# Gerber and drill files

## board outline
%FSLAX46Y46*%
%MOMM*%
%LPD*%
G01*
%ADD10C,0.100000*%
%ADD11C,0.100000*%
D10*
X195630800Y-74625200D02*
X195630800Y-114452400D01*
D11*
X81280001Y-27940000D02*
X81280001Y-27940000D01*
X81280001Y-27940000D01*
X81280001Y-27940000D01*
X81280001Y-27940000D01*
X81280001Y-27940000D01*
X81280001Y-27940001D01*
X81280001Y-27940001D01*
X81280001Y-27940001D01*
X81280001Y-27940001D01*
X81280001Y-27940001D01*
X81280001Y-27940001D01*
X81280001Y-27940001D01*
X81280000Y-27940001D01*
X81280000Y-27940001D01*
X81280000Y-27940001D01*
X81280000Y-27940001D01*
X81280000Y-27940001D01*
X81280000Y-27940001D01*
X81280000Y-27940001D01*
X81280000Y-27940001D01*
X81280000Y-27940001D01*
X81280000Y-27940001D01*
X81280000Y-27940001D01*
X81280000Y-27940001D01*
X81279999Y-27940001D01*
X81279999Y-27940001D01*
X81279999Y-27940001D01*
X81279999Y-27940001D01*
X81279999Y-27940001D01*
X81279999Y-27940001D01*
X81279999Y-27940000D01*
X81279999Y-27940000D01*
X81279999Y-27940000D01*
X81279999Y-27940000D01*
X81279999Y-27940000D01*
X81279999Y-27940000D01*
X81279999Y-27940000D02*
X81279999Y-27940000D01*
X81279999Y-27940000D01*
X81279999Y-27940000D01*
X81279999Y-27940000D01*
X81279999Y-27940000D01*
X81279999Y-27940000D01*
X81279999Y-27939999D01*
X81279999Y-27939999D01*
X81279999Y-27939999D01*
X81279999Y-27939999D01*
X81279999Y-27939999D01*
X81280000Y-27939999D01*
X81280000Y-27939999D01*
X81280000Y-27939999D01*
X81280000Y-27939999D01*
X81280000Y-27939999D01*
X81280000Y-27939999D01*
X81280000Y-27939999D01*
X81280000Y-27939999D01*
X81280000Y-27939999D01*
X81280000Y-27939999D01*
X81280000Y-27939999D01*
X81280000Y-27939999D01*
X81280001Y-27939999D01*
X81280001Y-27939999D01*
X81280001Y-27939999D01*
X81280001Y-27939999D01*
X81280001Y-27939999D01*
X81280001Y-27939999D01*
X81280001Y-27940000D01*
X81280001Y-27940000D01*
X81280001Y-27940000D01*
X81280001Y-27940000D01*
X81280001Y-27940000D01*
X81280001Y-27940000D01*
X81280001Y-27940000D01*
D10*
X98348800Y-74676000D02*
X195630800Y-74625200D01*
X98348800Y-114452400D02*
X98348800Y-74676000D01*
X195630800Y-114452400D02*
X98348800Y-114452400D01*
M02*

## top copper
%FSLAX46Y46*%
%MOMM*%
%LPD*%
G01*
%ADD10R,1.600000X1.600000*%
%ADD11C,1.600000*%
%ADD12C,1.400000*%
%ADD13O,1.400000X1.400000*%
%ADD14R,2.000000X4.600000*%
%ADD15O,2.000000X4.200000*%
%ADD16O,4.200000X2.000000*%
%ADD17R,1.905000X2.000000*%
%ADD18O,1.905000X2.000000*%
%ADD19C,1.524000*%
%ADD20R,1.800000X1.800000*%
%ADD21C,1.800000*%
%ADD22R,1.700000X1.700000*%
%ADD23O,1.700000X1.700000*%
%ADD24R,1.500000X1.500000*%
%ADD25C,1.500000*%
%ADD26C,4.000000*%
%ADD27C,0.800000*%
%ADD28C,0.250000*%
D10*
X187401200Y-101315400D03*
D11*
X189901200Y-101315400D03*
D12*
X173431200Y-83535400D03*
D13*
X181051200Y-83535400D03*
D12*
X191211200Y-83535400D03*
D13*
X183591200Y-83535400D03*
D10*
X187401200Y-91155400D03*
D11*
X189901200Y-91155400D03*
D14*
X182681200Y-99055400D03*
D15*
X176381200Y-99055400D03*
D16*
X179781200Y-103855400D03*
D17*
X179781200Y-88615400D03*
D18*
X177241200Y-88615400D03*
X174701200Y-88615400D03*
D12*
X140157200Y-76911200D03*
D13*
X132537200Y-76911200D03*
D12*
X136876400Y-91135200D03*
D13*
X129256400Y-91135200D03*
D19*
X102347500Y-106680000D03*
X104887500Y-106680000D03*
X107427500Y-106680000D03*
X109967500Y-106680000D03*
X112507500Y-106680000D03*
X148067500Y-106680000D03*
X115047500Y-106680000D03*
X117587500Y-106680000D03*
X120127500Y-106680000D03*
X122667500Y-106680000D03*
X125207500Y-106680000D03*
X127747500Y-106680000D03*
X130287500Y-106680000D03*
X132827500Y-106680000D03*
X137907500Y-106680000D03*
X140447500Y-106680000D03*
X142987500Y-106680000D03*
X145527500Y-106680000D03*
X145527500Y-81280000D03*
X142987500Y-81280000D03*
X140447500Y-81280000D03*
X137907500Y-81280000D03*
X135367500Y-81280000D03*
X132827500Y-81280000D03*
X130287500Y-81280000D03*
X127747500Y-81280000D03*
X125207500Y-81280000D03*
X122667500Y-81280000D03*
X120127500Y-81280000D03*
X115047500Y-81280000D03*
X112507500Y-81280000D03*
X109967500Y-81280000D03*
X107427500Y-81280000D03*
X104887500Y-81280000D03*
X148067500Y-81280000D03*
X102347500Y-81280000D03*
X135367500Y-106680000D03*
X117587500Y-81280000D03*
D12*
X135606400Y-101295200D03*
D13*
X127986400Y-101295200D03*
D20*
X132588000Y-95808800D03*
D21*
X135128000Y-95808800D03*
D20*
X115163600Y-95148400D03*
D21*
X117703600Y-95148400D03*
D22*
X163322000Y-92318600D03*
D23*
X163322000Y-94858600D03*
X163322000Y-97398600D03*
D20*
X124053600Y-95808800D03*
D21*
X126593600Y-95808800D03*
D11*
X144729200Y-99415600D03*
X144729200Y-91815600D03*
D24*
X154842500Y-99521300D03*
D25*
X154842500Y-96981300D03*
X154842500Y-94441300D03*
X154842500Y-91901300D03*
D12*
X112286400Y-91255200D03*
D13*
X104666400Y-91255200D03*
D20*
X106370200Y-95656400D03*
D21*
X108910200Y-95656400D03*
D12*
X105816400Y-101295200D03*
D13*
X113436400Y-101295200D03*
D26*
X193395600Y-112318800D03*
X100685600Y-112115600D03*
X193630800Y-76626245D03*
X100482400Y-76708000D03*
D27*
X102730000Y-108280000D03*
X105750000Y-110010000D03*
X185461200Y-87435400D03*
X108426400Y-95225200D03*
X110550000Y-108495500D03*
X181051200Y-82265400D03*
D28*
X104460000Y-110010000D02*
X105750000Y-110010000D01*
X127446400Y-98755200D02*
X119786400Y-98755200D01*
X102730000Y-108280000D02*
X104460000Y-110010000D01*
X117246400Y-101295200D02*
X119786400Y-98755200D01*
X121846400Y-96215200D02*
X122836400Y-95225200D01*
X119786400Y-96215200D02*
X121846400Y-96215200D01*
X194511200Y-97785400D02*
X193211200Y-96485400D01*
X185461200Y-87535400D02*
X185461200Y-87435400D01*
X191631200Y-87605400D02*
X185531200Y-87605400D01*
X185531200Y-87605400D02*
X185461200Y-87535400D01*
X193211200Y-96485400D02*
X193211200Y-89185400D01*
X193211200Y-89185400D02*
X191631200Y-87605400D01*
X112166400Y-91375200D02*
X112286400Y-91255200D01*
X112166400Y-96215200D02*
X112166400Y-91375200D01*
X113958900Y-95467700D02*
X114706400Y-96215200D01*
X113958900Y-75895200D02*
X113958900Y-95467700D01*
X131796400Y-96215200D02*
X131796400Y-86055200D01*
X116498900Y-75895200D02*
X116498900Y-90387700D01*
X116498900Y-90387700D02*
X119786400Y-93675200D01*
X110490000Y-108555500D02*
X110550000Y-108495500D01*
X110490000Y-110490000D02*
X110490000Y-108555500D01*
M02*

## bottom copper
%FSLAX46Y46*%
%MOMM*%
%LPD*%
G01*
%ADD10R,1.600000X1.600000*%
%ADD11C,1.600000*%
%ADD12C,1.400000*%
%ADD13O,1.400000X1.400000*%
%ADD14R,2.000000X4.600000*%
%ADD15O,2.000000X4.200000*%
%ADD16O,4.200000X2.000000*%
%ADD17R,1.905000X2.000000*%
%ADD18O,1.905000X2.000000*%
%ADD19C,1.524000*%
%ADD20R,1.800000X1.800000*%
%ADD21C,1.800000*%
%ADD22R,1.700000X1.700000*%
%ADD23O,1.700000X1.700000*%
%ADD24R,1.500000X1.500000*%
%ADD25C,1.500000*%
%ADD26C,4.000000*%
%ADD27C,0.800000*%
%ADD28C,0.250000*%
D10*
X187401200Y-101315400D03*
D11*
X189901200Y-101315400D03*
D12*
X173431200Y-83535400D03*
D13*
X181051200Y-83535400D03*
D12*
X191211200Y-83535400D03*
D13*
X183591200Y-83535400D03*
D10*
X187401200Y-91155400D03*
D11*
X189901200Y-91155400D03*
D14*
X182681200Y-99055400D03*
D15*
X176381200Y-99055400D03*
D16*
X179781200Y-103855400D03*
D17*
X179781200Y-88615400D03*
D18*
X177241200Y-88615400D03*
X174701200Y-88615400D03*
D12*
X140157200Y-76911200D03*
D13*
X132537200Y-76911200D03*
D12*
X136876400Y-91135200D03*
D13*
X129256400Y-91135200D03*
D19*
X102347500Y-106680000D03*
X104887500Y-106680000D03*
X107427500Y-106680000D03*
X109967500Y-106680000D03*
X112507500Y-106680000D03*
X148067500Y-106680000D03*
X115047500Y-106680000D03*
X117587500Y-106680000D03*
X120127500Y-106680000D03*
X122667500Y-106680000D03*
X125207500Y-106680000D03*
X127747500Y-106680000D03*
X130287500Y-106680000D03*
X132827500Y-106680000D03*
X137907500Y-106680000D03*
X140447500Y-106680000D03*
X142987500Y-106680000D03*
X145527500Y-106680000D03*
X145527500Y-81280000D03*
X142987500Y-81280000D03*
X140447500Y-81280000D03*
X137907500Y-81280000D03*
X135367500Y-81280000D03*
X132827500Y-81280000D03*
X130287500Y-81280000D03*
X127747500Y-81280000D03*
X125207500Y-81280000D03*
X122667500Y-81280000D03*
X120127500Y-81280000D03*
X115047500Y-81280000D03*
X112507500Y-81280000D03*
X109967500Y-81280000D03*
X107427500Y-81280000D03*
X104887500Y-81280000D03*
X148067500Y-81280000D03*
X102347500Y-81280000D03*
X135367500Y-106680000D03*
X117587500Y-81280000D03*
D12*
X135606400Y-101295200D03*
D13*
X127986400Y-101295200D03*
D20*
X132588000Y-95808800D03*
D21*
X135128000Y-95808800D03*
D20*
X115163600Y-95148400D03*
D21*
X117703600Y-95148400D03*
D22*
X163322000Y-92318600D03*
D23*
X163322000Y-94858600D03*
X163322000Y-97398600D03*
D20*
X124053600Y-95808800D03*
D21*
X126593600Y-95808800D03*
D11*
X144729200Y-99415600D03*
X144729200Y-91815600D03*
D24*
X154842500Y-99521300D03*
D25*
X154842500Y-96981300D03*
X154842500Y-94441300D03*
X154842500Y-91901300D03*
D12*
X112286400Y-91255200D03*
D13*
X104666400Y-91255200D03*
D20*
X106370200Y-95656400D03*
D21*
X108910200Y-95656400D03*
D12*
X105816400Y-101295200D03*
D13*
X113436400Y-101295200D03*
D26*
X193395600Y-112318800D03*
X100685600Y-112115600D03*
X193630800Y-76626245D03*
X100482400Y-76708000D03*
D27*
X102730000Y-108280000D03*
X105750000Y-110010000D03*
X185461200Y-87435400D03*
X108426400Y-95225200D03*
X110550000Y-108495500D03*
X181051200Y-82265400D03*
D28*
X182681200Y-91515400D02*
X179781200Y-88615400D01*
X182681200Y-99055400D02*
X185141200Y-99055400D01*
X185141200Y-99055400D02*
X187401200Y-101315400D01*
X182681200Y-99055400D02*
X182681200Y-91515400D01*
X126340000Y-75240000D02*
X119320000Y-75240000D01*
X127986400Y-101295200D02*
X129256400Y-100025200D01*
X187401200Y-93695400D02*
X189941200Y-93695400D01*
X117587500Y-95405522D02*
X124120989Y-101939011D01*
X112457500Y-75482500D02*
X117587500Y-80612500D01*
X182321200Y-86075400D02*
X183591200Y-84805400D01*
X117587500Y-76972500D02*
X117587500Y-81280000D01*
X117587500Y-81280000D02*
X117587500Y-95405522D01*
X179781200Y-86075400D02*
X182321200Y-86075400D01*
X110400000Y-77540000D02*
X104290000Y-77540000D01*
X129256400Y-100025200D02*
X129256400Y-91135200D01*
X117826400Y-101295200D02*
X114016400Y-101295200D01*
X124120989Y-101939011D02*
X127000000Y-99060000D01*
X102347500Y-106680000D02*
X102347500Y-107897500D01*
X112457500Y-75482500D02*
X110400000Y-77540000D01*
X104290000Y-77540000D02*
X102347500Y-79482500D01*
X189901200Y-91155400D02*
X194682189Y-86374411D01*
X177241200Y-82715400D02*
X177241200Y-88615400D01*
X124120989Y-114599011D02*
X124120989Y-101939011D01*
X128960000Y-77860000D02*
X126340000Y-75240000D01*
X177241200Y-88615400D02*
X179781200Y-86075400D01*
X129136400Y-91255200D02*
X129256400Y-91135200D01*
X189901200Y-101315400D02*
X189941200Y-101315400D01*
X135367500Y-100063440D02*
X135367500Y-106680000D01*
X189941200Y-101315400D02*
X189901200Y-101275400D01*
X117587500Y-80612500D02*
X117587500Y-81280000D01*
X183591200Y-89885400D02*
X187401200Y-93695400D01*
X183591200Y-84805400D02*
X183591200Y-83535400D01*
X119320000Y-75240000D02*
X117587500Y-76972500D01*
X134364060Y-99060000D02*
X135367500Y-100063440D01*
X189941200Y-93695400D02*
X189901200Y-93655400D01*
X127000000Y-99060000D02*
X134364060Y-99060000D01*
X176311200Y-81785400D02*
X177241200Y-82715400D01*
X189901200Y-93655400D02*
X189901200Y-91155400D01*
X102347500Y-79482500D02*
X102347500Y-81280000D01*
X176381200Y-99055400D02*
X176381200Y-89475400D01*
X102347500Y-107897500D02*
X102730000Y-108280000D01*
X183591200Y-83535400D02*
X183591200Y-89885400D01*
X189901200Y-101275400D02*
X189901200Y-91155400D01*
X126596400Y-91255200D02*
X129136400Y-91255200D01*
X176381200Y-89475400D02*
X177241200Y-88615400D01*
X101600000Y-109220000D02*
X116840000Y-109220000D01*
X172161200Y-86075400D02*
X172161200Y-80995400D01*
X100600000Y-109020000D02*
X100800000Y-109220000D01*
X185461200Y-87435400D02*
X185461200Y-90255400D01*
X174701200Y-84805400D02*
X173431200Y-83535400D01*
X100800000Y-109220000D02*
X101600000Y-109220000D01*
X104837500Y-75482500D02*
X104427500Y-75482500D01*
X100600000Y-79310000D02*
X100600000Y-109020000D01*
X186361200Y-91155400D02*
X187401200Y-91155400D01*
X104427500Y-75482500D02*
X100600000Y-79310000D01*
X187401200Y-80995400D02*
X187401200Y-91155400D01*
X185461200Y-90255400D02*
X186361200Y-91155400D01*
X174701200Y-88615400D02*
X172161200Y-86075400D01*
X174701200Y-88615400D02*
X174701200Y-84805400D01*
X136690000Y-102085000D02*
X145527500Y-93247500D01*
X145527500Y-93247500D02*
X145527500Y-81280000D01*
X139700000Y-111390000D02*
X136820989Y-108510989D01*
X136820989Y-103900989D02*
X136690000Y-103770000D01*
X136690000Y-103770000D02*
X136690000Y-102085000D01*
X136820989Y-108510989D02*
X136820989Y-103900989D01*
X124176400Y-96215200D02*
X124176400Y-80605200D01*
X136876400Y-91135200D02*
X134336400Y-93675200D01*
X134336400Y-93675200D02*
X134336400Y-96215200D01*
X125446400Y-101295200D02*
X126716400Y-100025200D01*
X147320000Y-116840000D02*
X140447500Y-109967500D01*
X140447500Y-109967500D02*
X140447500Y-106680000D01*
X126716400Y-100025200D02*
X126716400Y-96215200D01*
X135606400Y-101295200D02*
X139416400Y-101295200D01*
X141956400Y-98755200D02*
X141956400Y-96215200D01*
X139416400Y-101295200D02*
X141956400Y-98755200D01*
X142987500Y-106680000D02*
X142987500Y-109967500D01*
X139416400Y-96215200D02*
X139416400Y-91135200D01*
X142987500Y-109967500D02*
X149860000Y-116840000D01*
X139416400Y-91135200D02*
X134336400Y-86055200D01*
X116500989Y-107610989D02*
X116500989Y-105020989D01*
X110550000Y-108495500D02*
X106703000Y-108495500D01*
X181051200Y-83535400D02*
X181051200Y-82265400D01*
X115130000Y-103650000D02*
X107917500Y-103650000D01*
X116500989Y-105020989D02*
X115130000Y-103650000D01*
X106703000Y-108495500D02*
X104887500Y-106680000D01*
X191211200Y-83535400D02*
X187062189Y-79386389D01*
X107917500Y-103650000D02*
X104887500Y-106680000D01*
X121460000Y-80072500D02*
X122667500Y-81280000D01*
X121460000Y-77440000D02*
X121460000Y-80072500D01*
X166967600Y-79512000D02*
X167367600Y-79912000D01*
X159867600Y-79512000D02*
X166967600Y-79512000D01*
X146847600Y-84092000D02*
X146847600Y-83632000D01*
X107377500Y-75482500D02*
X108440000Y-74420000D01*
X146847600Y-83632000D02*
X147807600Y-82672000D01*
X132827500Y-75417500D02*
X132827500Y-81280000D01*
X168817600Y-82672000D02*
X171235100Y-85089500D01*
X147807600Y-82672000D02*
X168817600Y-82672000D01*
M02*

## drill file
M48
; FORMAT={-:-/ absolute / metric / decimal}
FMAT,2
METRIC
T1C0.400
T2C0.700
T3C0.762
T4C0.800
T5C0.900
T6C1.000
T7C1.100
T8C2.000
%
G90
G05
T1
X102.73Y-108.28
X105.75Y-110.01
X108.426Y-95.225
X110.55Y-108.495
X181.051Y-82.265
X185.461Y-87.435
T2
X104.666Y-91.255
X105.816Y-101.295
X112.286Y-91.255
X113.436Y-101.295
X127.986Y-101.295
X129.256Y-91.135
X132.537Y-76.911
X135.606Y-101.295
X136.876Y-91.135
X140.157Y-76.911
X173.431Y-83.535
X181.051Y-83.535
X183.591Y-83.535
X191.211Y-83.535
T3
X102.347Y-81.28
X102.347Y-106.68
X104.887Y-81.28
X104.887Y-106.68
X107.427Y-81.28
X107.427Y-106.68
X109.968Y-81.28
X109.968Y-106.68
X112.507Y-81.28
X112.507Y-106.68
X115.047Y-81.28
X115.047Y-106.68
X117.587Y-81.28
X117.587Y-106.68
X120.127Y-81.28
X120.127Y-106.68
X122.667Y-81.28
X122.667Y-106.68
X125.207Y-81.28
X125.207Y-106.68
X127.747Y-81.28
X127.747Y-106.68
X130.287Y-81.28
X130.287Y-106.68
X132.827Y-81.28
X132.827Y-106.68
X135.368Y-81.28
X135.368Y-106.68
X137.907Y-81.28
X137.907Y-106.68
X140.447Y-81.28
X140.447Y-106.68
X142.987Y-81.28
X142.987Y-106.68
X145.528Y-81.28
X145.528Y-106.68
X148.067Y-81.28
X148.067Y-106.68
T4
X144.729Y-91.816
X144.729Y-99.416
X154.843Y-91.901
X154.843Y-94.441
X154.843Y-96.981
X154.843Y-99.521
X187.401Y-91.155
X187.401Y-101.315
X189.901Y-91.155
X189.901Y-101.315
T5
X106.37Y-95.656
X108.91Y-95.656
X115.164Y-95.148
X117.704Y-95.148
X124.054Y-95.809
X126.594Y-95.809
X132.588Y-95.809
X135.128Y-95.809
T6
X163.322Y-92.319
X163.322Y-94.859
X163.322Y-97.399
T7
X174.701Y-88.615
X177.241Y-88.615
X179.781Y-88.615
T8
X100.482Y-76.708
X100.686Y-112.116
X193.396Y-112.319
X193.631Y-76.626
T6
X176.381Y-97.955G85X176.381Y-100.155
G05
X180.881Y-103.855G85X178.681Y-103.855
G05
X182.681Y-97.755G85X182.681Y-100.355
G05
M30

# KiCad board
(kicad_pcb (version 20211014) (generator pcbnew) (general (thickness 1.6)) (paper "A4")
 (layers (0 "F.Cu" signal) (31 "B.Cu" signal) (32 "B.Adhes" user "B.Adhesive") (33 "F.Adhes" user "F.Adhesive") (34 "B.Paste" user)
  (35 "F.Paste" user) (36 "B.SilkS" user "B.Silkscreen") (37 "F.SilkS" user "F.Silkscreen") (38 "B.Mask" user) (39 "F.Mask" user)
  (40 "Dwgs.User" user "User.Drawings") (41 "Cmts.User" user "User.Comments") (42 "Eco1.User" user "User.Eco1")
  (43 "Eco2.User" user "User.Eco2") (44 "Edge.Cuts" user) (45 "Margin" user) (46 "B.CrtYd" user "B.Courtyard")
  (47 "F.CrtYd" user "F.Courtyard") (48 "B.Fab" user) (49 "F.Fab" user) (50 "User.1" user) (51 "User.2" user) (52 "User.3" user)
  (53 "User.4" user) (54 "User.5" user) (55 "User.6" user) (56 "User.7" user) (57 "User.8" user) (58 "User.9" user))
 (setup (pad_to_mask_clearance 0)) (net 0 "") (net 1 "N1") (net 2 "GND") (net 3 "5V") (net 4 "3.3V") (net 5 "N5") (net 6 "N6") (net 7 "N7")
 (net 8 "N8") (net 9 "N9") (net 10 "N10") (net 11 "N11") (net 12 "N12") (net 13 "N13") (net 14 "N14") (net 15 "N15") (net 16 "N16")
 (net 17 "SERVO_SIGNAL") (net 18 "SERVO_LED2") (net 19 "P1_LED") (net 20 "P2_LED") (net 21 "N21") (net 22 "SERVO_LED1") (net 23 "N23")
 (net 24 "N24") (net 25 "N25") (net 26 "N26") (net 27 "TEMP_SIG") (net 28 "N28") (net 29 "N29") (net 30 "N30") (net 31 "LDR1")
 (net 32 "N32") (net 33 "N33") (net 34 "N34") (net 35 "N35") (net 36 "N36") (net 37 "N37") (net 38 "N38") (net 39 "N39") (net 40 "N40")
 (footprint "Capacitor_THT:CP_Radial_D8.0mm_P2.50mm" (layer "F.Cu") (at 187.4012 101.3154)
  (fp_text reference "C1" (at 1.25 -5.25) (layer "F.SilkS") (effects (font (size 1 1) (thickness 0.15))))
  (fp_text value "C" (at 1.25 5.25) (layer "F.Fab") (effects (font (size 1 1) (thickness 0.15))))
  (pad "1" thru_hole rect (at 0 0) (size 1.6 1.6) (drill 0.8) (layers *.Cu *.Mask) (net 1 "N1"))
  (pad "2" thru_hole circle (at 2.5 0) (size 1.6 1.6) (drill 0.8) (layers *.Cu *.Mask) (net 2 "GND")))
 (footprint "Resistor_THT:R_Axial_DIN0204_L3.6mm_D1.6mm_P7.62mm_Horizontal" (layer "F.Cu") (at 173.4312 83.5354)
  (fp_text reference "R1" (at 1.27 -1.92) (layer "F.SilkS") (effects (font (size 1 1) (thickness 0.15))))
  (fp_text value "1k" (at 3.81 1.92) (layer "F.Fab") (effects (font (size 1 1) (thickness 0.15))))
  (pad "1" thru_hole circle (at 0 0) (size 1.4 1.4) (drill 0.7) (layers *.Cu *.Mask) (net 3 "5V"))
  (pad "2" thru_hole oval (at 7.62 0) (size 1.4 1.4) (drill 0.7) (layers *.Cu *.Mask) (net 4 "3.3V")))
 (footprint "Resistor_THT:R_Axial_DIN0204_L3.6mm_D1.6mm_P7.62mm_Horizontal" (layer "F.Cu") (at 191.2112 83.5354 180)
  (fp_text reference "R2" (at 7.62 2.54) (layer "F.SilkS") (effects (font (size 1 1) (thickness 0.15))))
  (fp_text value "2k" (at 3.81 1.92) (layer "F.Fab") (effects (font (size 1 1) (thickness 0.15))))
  (pad "1" thru_hole circle (at 0 0 180) (size 1.4 1.4) (drill 0.7) (layers *.Cu *.Mask) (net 4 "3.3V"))
  (pad "2" thru_hole oval (at 7.62 0 180) (size 1.4 1.4) (drill 0.7) (layers *.Cu *.Mask) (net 2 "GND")))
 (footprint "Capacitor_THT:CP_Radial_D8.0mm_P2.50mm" (layer "F.Cu") (at 187.4012 91.1554)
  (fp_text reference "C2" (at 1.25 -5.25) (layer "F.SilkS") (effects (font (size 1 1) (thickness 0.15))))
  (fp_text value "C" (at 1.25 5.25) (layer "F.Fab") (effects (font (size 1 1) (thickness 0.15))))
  (pad "1" thru_hole rect (at 0 0) (size 1.6 1.6) (drill 0.8) (layers *.Cu *.Mask) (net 3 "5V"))
  (pad "2" thru_hole circle (at 2.5 0) (size 1.6 1.6) (drill 0.8) (layers *.Cu *.Mask) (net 2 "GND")))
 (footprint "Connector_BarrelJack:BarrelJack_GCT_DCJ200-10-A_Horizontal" (layer "F.Cu") (at 182.6812 99.0554 -90)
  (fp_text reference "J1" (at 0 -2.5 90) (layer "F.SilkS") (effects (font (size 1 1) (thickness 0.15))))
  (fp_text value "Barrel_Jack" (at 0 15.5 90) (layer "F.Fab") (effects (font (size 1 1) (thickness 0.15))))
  (pad "1" thru_hole rect (at 0 0 270) (size 4.6 2) (drill oval 3.6 1) (layers *.Cu *.Mask) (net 1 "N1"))
  (pad "2" thru_hole oval (at 0 6.3 270) (size 4.2 2) (drill oval 3.2 1) (layers *.Cu *.Mask) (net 2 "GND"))
  (pad "3" thru_hole oval (at 4.8 2.9 270) (size 2 4.2) (drill oval 1 3.2) (layers *.Cu *.Mask)))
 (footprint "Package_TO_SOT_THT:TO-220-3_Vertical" (layer "F.Cu") (at 179.7812 88.6154 180)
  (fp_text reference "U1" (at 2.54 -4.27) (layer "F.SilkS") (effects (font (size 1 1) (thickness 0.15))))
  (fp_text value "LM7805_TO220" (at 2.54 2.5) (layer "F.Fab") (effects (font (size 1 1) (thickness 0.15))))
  (pad "1" thru_hole rect (at 0 0 180) (size 1.905 2) (drill 1.1) (layers *.Cu *.Mask) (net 1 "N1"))
  (pad "2" thru_hole oval (at 2.54 0 180) (size 1.905 2) (drill 1.1) (layers *.Cu *.Mask) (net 2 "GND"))
  (pad "3" thru_hole oval (at 5.08 0 180) (size 1.905 2) (drill 1.1) (layers *.Cu *.Mask) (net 3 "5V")))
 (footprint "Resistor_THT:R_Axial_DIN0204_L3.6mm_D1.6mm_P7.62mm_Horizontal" (layer "F.Cu") (at 140.1572 76.9112 180)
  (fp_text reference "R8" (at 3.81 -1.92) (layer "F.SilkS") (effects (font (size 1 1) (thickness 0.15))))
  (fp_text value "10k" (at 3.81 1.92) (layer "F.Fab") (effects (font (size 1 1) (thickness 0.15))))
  (pad "1" thru_hole circle (at 0 0 180) (size 1.4 1.4) (drill 0.7) (layers *.Cu *.Mask) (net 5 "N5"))
  (pad "2" thru_hole oval (at 7.62 0 180) (size 1.4 1.4) (drill 0.7) (layers *.Cu *.Mask) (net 2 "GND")))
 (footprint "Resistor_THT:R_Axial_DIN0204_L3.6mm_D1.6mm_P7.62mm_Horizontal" (layer "F.Cu") (at 136.8764 91.1352 180)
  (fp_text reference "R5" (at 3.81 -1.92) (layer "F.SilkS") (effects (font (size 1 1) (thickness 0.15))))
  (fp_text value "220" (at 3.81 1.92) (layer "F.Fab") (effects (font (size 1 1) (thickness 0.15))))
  (pad "1" thru_hole circle (at 0 0 180) (size 1.4 1.4) (drill 0.7) (layers *.Cu *.Mask) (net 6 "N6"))
  (pad "2" thru_hole oval (at 7.62 0 180) (size 1.4 1.4) (drill 0.7) (layers *.Cu *.Mask) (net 2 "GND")))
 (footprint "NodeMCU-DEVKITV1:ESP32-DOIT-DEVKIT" (layer "F.Cu") (at 99.8075 93.98 90)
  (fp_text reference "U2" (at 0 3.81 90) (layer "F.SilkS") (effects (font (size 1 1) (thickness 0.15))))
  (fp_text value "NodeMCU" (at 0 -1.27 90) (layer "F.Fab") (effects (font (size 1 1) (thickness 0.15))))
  (pad "1" thru_hole circle (at -12.7 2.54 90) (size 1.524 1.524) (drill 0.762) (layers *.Cu *.Mask) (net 2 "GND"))
  (pad "2" thru_hole circle (at -12.7 5.08 90) (size 1.524 1.524) (drill 0.762) (layers *.Cu *.Mask) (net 4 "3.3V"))
  (pad "3" thru_hole circle (at -12.7 7.62 90) (size 1.524 1.524) (drill 0.762) (layers *.Cu *.Mask) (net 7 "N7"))
  (pad "4" thru_hole circle (at -12.7 10.16 90) (size 1.524 1.524) (drill 0.762) (layers *.Cu *.Mask) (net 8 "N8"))
  (pad "5" thru_hole circle (at -12.7 12.7 90) (size 1.524 1.524) (drill 0.762) (layers *.Cu *.Mask) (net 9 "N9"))
  (pad "5V" thru_hole circle (at -12.7 48.26 90) (size 1.524 1.524) (drill 0.762) (layers *.Cu *.Mask) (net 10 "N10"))
  (pad "6" thru_hole circle (at -12.7 15.24 90) (size 1.524 1.524) (drill 0.762) (layers *.Cu *.Mask) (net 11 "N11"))
  (pad "7" thru_hole circle (at -12.7 17.78 90) (size 1.524 1.524) (drill 0.762) (layers *.Cu *.Mask) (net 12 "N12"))
  (pad "8" thru_hole circle (at -12.7 20.32 90) (size 1.524 1.524) (drill 0.762) (layers *.Cu *.Mask) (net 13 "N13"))
  (pad "9" thru_hole circle (at -12.7 22.86 90) (size 1.524 1.524) (drill 0.762) (layers *.Cu *.Mask) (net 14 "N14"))
  (pad "10" thru_hole circle (at -12.7 25.4 90) (size 1.524 1.524) (drill 0.762) (layers *.Cu *.Mask) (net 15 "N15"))
  (pad "11" thru_hole circle (at -12.7 27.94 90) (size 1.524 1.524) (drill 0.762) (layers *.Cu *.Mask) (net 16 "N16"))
  (pad "12" thru_hole circle (at -12.7 30.48 90) (size 1.524 1.524) (drill 0.762) (layers *.Cu *.Mask) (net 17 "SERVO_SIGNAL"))
  (pad "13" thru_hole circle (at -12.7 33.02 90) (size 1.524 1.524) (drill 0.762) (layers *.Cu *.Mask) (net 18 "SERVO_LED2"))
  (pad "15" thru_hole circle (at -12.7 38.1 90) (size 1.524 1.524) (drill 0.762) (layers *.Cu *.Mask))
  (pad "16" thru_hole circle (at -12.7 40.64 90) (size 1.524 1.524) (drill 0.762) (layers *.Cu *.Mask) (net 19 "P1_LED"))
  (pad "17" thru_hole circle (at -12.7 43.18 90) (size 1.524 1.524) (drill 0.762) (layers *.Cu *.Mask) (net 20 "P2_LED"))
  (pad "18" thru_hole circle (at -12.7 45.72 90) (size 1.524 1.524) (drill 0.762) (layers *.Cu *.Mask) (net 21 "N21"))
  (pad "19" thru_hole circle (at 12.7 45.72 90) (size 1.524 1.524) (drill 0.762) (layers *.Cu *.Mask) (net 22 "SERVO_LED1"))
  (pad "20" thru_hole circle (at 12.7 43.18 90) (size 1.524 1.524) (drill 0.762) (layers *.Cu *.Mask) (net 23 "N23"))
  (pad "21" thru_hole circle (at 12.7 40.64 90) (size 1.524 1.524) (drill 0.762) (layers *.Cu *.Mask) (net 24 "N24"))
  (pad "22" thru_hole circle (at 12.7 38.1 90) (size 1.524 1.524) (drill 0.762) (layers *.Cu *.Mask) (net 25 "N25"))
  (pad "23" thru_hole circle (at 12.7 35.56 90) (size 1.524 1.524) (drill 0.762) (layers *.Cu *.Mask) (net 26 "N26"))
  (pad "24" thru_hole circle (at 12.7 33.02 90) (size 1.524 1.524) (drill 0.762) (layers *.Cu *.Mask) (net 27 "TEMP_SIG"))
  (pad "25" thru_hole circle (at 12.7 30.48 90) (size 1.524 1.524) (drill 0.762) (layers *.Cu *.Mask) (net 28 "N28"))
  (pad "26" thru_hole circle (at 12.7 27.94 90) (size 1.524 1.524) (drill 0.762) (layers *.Cu *.Mask) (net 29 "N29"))
  (pad "27" thru_hole circle (at 12.7 25.4 90) (size 1.524 1.524) (drill 0.762) (layers *.Cu *.Mask) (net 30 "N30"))
  (pad "28" thru_hole circle (at 12.7 22.86 90) (size 1.524 1.524) (drill 0.762) (layers *.Cu *.Mask) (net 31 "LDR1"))
  (pad "29" thru_hole circle (at 12.7 20.32 90) (size 1.524 1.524) (drill 0.762) (layers *.Cu *.Mask) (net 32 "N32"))
  (pad "31" thru_hole circle (at 12.7 15.24 90) (size 1.524 1.524) (drill 0.762) (layers *.Cu *.Mask) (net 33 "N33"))
  (pad "32" thru_hole circle (at 12.7 12.7 90) (size 1.524 1.524) (drill 0.762) (layers *.Cu *.Mask))
  (pad "33" thru_hole circle (at 12.7 10.16 90) (size 1.524 1.524) (drill 0.762) (layers *.Cu *.Mask) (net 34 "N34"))
  (pad "34" thru_hole circle (at 12.7 7.62 90) (size 1.524 1.524) (drill 0.762) (layers *.Cu *.Mask) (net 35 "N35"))
  (pad "35" thru_hole circle (at 12.7 5.08 90) (size 1.524 1.524) (drill 0.762) (layers *.Cu *.Mask) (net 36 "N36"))
  (pad "38" thru_hole circle (at 12.7 48.26 90) (size 1.524 1.524) (drill 0.762) (layers *.Cu *.Mask))
  (pad "GND" thru_hole circle (at 12.7 2.54 90) (size 1.524 1.524) (drill 0.762) (layers *.Cu *.Mask) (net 2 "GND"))
  (pad "GND" thru_hole circle (at -12.7 35.56 90) (size 1.524 1.524) (drill 0.762) (layers *.Cu *.Mask) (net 2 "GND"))
  (pad "GND" thru_hole circle (at 12.7 17.78 90) (size 1.524 1.524) (drill 0.762) (layers *.Cu *.Mask) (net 2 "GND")))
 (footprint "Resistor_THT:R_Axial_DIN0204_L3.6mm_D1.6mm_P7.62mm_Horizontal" (layer "F.Cu") (at 135.6064 101.2952 180)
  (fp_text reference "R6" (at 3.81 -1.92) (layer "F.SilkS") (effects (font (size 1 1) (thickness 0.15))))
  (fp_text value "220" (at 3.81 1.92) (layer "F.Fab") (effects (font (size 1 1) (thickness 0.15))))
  (pad "1" thru_hole circle (at 0 0 180) (size 1.4 1.4) (drill 0.7) (layers *.Cu *.Mask) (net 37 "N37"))
  (pad "2" thru_hole oval (at 7.62 0 180) (size 1.4 1.4) (drill 0.7) (layers *.Cu *.Mask) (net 2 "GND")))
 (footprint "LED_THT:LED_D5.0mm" (layer "B.Cu") (at 132.588 95.8088)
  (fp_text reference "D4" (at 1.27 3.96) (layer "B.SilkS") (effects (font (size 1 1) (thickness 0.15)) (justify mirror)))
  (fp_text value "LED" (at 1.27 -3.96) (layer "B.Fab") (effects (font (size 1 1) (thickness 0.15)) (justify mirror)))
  (pad "1" thru_hole rect (at 0 0) (size 1.8 1.8) (drill 0.9) (layers *.Cu *.Mask) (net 37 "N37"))
  (pad "2" thru_hole circle (at 2.54 0) (size 1.8 1.8) (drill 0.9) (layers *.Cu *.Mask) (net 20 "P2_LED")))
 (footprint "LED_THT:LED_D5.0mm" (layer "B.Cu") (at 115.1636 95.1484)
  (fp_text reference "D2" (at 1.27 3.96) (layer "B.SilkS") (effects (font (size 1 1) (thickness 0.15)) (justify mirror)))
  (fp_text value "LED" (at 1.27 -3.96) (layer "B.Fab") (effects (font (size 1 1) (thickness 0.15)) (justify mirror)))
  (pad "1" thru_hole rect (at 0 0) (size 1.8 1.8) (drill 0.9) (layers *.Cu *.Mask) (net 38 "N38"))
  (pad "2" thru_hole circle (at 2.54 0) (size 1.8 1.8) (drill 0.9) (layers *.Cu *.Mask) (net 22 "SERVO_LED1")))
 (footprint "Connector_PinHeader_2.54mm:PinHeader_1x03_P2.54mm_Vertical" (layer "B.Cu") (at 163.322 92.3186 180)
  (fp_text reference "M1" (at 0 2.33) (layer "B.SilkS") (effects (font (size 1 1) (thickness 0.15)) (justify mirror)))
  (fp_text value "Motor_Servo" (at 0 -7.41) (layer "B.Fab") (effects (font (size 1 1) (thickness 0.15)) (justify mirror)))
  (pad "1" thru_hole rect (at 0 0 180) (size 1.7 1.7) (drill 1) (layers *.Cu *.Mask) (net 17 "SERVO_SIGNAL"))
  (pad "2" thru_hole oval (at 0 -2.54 180) (size 1.7 1.7) (drill 1) (layers *.Cu *.Mask) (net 3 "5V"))
  (pad "3" thru_hole oval (at 0 -5.08 180) (size 1.7 1.7) (drill 1) (layers *.Cu *.Mask) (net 2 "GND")))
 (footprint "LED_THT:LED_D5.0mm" (layer "B.Cu") (at 124.0536 95.8088)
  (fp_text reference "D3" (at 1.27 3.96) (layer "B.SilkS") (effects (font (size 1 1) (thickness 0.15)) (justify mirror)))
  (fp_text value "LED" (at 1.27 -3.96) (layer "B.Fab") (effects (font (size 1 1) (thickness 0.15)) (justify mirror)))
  (pad "1" thru_hole rect (at 0 0) (size 1.8 1.8) (drill 0.9) (layers *.Cu *.Mask) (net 6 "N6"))
  (pad "2" thru_hole circle (at 2.54 0) (size 1.8 1.8) (drill 0.9) (layers *.Cu *.Mask) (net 19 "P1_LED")))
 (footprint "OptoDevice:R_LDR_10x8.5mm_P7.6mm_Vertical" (layer "B.Cu") (at 144.7292 99.4156 90)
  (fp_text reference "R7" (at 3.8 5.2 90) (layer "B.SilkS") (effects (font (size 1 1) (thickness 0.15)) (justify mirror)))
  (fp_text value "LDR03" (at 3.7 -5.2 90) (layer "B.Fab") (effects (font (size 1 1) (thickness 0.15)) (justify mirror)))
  (pad "1" thru_hole circle (at 0 0 90) (size 1.6 1.6) (drill 0.8) (layers *.Cu *.Mask) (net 31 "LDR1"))
  (pad "2" thru_hole circle (at 7.6 0 90) (size 1.6 1.6) (drill 0.8) (layers *.Cu *.Mask) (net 5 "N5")))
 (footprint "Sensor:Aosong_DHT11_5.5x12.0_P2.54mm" (layer "B.Cu") (at 154.8425 99.5213)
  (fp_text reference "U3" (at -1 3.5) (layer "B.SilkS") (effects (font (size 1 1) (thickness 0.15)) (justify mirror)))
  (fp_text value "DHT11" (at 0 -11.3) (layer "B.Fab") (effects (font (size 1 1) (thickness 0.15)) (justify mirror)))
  (pad "1" thru_hole rect (at 0 0) (size 1.5 1.5) (drill 0.8) (layers *.Cu *.Mask) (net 3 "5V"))
  (pad "2" thru_hole circle (at 0 -2.54) (size 1.5 1.5) (drill 0.8) (layers *.Cu *.Mask) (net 27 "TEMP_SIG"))
  (pad "3" thru_hole circle (at 0 -5.08) (size 1.5 1.5) (drill 0.8) (layers *.Cu *.Mask) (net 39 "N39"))
  (pad "4" thru_hole circle (at 0 -7.62) (size 1.5 1.5) (drill 0.8) (layers *.Cu *.Mask) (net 2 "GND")))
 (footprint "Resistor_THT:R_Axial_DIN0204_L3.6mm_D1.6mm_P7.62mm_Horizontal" (layer "B.Cu") (at 112.2864 91.2552 180)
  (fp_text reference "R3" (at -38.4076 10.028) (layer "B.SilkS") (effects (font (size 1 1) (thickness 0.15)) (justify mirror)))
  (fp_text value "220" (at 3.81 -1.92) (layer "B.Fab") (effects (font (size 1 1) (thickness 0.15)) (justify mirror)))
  (pad "1" thru_hole circle (at 0 0 180) (size 1.4 1.4) (drill 0.7) (layers *.Cu *.Mask) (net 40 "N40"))
  (pad "2" thru_hole oval (at 7.62 0 180) (size 1.4 1.4) (drill 0.7) (layers *.Cu *.Mask) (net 2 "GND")))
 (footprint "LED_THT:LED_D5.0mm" (layer "B.Cu") (at 106.3702 95.6564)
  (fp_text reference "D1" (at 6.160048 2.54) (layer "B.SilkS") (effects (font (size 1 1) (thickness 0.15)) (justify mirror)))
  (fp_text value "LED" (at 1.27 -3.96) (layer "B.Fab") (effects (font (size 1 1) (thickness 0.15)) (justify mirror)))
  (pad "1" thru_hole rect (at 0 0) (size 1.8 1.8) (drill 0.9) (layers *.Cu *.Mask) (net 40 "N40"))
  (pad "2" thru_hole circle (at 2.54 0) (size 1.8 1.8) (drill 0.9) (layers *.Cu *.Mask) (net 18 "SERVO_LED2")))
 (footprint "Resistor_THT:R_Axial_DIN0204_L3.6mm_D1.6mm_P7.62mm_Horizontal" (layer "B.Cu") (at 105.8164 101.2952)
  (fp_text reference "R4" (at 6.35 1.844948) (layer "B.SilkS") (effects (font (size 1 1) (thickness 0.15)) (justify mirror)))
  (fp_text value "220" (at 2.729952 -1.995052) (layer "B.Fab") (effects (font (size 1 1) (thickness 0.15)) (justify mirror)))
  (pad "1" thru_hole circle (at 0 0) (size 1.4 1.4) (drill 0.7) (layers *.Cu *.Mask) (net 38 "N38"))
  (pad "2" thru_hole oval (at 7.62 0) (size 1.4 1.4) (drill 0.7) (layers *.Cu *.Mask) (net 2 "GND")))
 (gr_line (start 195.6308 74.6252) (end 195.6308 114.4524) (layer "Edge.Cuts") (width 0.1))
 (gr_arc (start 81.28 27.94) (mid 81.28 27.94) (end 81.28 27.94) (layer "Edge.Cuts") (width 0.1))
 (gr_line (start 98.3488 74.676) (end 195.6308 74.6252) (layer "Edge.Cuts") (width 0.1))
 (gr_line (start 98.3488 114.4524) (end 98.3488 74.676) (layer "Edge.Cuts") (width 0.1))
 (gr_line (start 195.6308 114.4524) (end 98.3488 114.4524) (layer "Edge.Cuts") (width 0.1))
 (via (at 193.3956 112.3188) (size 4) (drill 2) (layers "F.Cu" "B.Cu") (free) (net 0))
 (via (at 100.6856 112.1156) (size 4) (drill 2) (layers "F.Cu" "B.Cu") (free) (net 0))
 (via (at 193.6308 76.626245) (size 4) (drill 2) (layers "F.Cu" "B.Cu") (free) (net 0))
 (via (at 100.4824 76.708) (size 4) (drill 2) (layers "F.Cu" "B.Cu") (free) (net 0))
 (segment (start 182.6812 91.5154) (end 179.7812 88.6154) (width 0.25) (layer "B.Cu") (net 1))
 (segment (start 182.6812 99.0554) (end 185.1412 99.0554) (width 0.25) (layer "B.Cu") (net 1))
 (segment (start 185.1412 99.0554) (end 187.4012 101.3154) (width 0.25) (layer "B.Cu") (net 1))
 (segment (start 182.6812 99.0554) (end 182.6812 91.5154) (width 0.25) (layer "B.Cu") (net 1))
 (segment (start 104.46 110.01) (end 105.75 110.01) (width 0.25) (layer "F.Cu") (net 2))
 (segment (start 127.4464 98.7552) (end 119.7864 98.7552) (width 0.25) (layer "F.Cu") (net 2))
 (segment (start 102.73 108.28) (end 104.46 110.01) (width 0.25) (layer "F.Cu") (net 2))
 (segment (start 117.2464 101.2952) (end 119.7864 98.7552) (width 0.25) (layer "F.Cu") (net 2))
 (via (at 102.73 108.28) (size 0.8) (drill 0.4) (layers "F.Cu" "B.Cu") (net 2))
 (via (at 105.75 110.01) (size 0.8) (drill 0.4) (layers "F.Cu" "B.Cu") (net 2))
 (segment (start 126.34 75.24) (end 119.32 75.24) (width 0.25) (layer "B.Cu") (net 2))
 (segment (start 127.9864 101.2952) (end 129.2564 100.0252) (width 0.25) (layer "B.Cu") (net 2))
 (segment (start 187.4012 93.6954) (end 189.9412 93.6954) (width 0.25) (layer "B.Cu") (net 2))
 (segment (start 117.5875 95.405522) (end 124.120989 101.939011) (width 0.25) (layer "B.Cu") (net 2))
 (segment (start 112.4575 75.4825) (end 117.5875 80.6125) (width 0.25) (layer "B.Cu") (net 2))
 (segment (start 182.3212 86.0754) (end 183.5912 84.8054) (width 0.25) (layer "B.Cu") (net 2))
 (segment (start 117.5875 76.9725) (end 117.5875 81.28) (width 0.25) (layer "B.Cu") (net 2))
 (segment (start 117.5875 81.28) (end 117.5875 95.405522) (width 0.25) (layer "B.Cu") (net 2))
 (segment (start 179.7812 86.0754) (end 182.3212 86.0754) (width 0.25) (layer "B.Cu") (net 2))
 (segment (start 110.4 77.54) (end 104.29 77.54) (width 0.25) (layer "B.Cu") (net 2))
 (segment (start 129.2564 100.0252) (end 129.2564 91.1352) (width 0.25) (layer "B.Cu") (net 2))
 (segment (start 117.8264 101.2952) (end 114.0164 101.2952) (width 0.25) (layer "B.Cu") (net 2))
 (segment (start 124.120989 101.939011) (end 127 99.06) (width 0.25) (layer "B.Cu") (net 2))
 (segment (start 102.3475 106.68) (end 102.3475 107.8975) (width 0.25) (layer "B.Cu") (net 2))
 (segment (start 112.4575 75.4825) (end 110.4 77.54) (width 0.25) (layer "B.Cu") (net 2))
 (segment (start 104.29 77.54) (end 102.3475 79.4825) (width 0.25) (layer "B.Cu") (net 2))
 (segment (start 189.9012 91.1554) (end 194.682189 86.374411) (width 0.25) (layer "B.Cu") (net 2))
 (segment (start 177.2412 82.7154) (end 177.2412 88.6154) (width 0.25) (layer "B.Cu") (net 2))
 (segment (start 124.120989 114.599011) (end 124.120989 101.939011) (width 0.25) (layer "B.Cu") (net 2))
 (segment (start 128.96 77.86) (end 126.34 75.24) (width 0.25) (layer "B.Cu") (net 2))
 (segment (start 177.2412 88.6154) (end 179.7812 86.0754) (width 0.25) (layer "B.Cu") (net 2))
 (segment (start 129.1364 91.2552) (end 129.2564 91.1352) (width 0.25) (layer "B.Cu") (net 2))
 (segment (start 189.9012 101.3154) (end 189.9412 101.3154) (width 0.25) (layer "B.Cu") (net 2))
 (segment (start 135.3675 100.06344) (end 135.3675 106.68) (width 0.25) (layer "B.Cu") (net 2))
 (segment (start 189.9412 101.3154) (end 189.9012 101.2754) (width 0.25) (layer "B.Cu") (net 2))
 (segment (start 117.5875 80.6125) (end 117.5875 81.28) (width 0.25) (layer "B.Cu") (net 2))
 (segment (start 183.5912 89.8854) (end 187.4012 93.6954) (width 0.25) (layer "B.Cu") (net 2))
 (segment (start 183.5912 84.8054) (end 183.5912 83.5354) (width 0.25) (layer "B.Cu") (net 2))
 (segment (start 119.32 75.24) (end 117.5875 76.9725) (width 0.25) (layer "B.Cu") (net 2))
 (segment (start 134.36406 99.06) (end 135.3675 100.06344) (width 0.25) (layer "B.Cu") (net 2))
 (segment (start 189.9412 93.6954) (end 189.9012 93.6554) (width 0.25) (layer "B.Cu") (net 2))
 (segment (start 127 99.06) (end 134.36406 99.06) (width 0.25) (layer "B.Cu") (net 2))
 (segment (start 176.3112 81.7854) (end 177.2412 82.7154) (width 0.25) (layer "B.Cu") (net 2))
 (segment (start 189.9012 93.6554) (end 189.9012 91.1554) (width 0.25) (layer "B.Cu") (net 2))
 (segment (start 102.3475 79.4825) (end 102.3475 81.28) (width 0.25) (layer "B.Cu") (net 2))
 (segment (start 176.3812 99.0554) (end 176.3812 89.4754) (width 0.25) (layer "B.Cu") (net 2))
 (segment (start 102.3475 107.8975) (end 102.73 108.28) (width 0.25) (layer "B.Cu") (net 2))
 (segment (start 183.5912 83.5354) (end 183.5912 89.8854) (width 0.25) (layer "B.Cu") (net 2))
 (segment (start 189.9012 101.2754) (end 189.9012 91.1554) (width 0.25) (layer "B.Cu") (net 2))
 (segment (start 126.5964 91.2552) (end 129.1364 91.2552) (width 0.25) (layer "B.Cu") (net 2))
 (segment (start 176.3812 89.4754) (end 177.2412 88.6154) (width 0.25) (layer "B.Cu") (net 2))
 (segment (start 121.8464 96.2152) (end 122.8364 95.2252) (width 0.25) (layer "F.Cu") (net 3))
 (segment (start 119.7864 96.2152) (end 121.8464 96.2152) (width 0.25) (layer "F.Cu") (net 3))
 (segment (start 194.5112 97.7854) (end 193.2112 96.4854) (width 0.25) (layer "F.Cu") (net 3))
 (segment (start 185.4612 87.5354) (end 185.4612 87.4354) (width 0.25) (layer "F.Cu") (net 3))
 (segment (start 191.6312 87.6054) (end 185.5312 87.6054) (width 0.25) (layer "F.Cu") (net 3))
 (segment (start 185.5312 87.6054) (end 185.4612 87.5354) (width 0.25) (layer "F.Cu") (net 3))
 (segment (start 193.2112 96.4854) (end 193.2112 89.1854) (width 0.25) (layer "F.Cu") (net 3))
 (segment (start 193.2112 89.1854) (end 191.6312 87.6054) (width 0.25) (layer "F.Cu") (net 3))
 (via (at 185.4612 87.4354) (size 0.8) (drill 0.4) (layers "F.Cu" "B.Cu") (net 3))
 (segment (start 101.6 109.22) (end 116.84 109.22) (width 0.25) (layer "B.Cu") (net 3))
 (segment (start 172.1612 86.0754) (end 172.1612 80.9954) (width 0.25) (layer "B.Cu") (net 3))
 (segment (start 100.6 109.02) (end 100.8 109.22) (width 0.25) (layer "B.Cu") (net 3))
 (segment (start 185.4612 87.4354) (end 185.4612 90.2554) (width 0.25) (layer "B.Cu") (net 3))
 (segment (start 174.7012 84.8054) (end 173.4312 83.5354) (width 0.25) (layer "B.Cu") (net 3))
 (segment (start 100.8 109.22) (end 101.6 109.22) (width 0.25) (layer "B.Cu") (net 3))
 (segment (start 104.8375 75.4825) (end 104.4275 75.4825) (width 0.25) (layer "B.Cu") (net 3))
 (segment (start 100.6 79.31) (end 100.6 109.02) (width 0.25) (layer "B.Cu") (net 3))
 (segment (start 186.3612 91.1554) (end 187.4012 91.1554) (width 0.25) (layer "B.Cu") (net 3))
 (segment (start 104.4275 75.4825) (end 100.6 79.31) (width 0.25) (layer "B.Cu") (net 3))
 (segment (start 187.4012 80.9954) (end 187.4012 91.1554) (width 0.25) (layer "B.Cu") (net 3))
 (segment (start 185.4612 90.2554) (end 186.3612 91.1554) (width 0.25) (layer "B.Cu") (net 3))
 (segment (start 174.7012 88.6154) (end 172.1612 86.0754) (width 0.25) (layer "B.Cu") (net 3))
 (segment (start 174.7012 88.6154) (end 174.7012 84.8054) (width 0.25) (layer "B.Cu") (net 3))
 (segment (start 112.1664 91.3752) (end 112.2864 91.2552) (width 0.25) (layer "F.Cu") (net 40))
 (segment (start 112.1664 96.2152) (end 112.1664 91.3752) (width 0.25) (layer "F.Cu") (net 40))
 (segment (start 113.9589 95.4677) (end 114.7064 96.2152) (width 0.25) (layer "F.Cu") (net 18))
 (segment (start 113.9589 75.8952) (end 113.9589 95.4677) (width 0.25) (layer "F.Cu") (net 18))
 (via (at 108.4264 95.2252) (size 0.8) (drill 0.4) (layers "F.Cu" "B.Cu") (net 18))
 (segment (start 136.69 102.085) (end 145.5275 93.2475) (width 0.25) (layer "B.Cu") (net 22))
 (segment (start 145.5275 93.2475) (end 145.5275 81.28) (width 0.25) (layer "B.Cu") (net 22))
 (segment (start 139.7 111.39) (end 136.820989 108.510989) (width 0.25) (layer "B.Cu") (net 22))
 (segment (start 136.820989 103.900989) (end 136.69 103.77) (width 0.25) (layer "B.Cu") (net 22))
 (segment (start 136.69 103.77) (end 136.69 102.085) (width 0.25) (layer "B.Cu") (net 22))
 (segment (start 136.820989 108.510989) (end 136.820989 103.900989) (width 0.25) (layer "B.Cu") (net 22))
 (segment (start 124.1764 96.2152) (end 124.1764 80.6052) (width 0.25) (layer "B.Cu") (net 6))
 (segment (start 136.8764 91.1352) (end 134.3364 93.6752) (width 0.25) (layer "B.Cu") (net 6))
 (segment (start 134.3364 93.6752) (end 134.3364 96.2152) (width 0.25) (layer "B.Cu") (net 6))
 (segment (start 125.4464 101.2952) (end 126.7164 100.0252) (width 0.25) (layer "B.Cu") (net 19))
 (segment (start 147.32 116.84) (end 140.4475 109.9675) (width 0.25) (layer "B.Cu") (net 19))
 (segment (start 140.4475 109.9675) (end 140.4475 106.68) (width 0.25) (layer "B.Cu") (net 19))
 (segment (start 126.7164 100.0252) (end 126.7164 96.2152) (width 0.25) (layer "B.Cu") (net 19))
 (segment (start 131.7964 96.2152) (end 131.7964 86.0552) (width 0.25) (layer "F.Cu") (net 37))
 (segment (start 135.6064 101.2952) (end 139.4164 101.2952) (width 0.25) (layer "B.Cu") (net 37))
 (segment (start 141.9564 98.7552) (end 141.9564 96.2152) (width 0.25) (layer "B.Cu") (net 37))
 (segment (start 139.4164 101.2952) (end 141.9564 98.7552) (width 0.25) (layer "B.Cu") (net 37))
 (segment (start 142.9875 106.68) (end 142.9875 109.9675) (width 0.25) (layer "B.Cu") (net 20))
 (segment (start 139.4164 96.2152) (end 139.4164 91.1352) (width 0.25) (layer "B.Cu") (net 20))
 (segment (start 142.9875 109.9675) (end 149.86 116.84) (width 0.25) (layer "B.Cu") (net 20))
 (segment (start 139.4164 91.1352) (end 134.3364 86.0552) (width 0.25) (layer "B.Cu") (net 20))
 (segment (start 116.4989 75.8952) (end 116.4989 90.3877) (width 0.25) (layer "F.Cu") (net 17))
 (segment (start 116.4989 90.3877) (end 119.7864 93.6752) (width 0.25) (layer "F.Cu") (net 17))
 (segment (start 110.49 108.5555) (end 110.55 108.4955) (width 0.25) (layer "F.Cu") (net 4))
 (segment (start 110.49 110.49) (end 110.49 108.5555) (width 0.25) (layer "F.Cu") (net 4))
 (via (at 110.55 108.4955) (size 0.8) (drill 0.4) (layers "F.Cu" "B.Cu") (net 4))
 (via (at 181.0512 82.2654) (size 0.8) (drill 0.4) (layers "F.Cu" "B.Cu") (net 4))
 (segment (start 116.500989 107.610989) (end 116.500989 105.020989) (width 0.25) (layer "B.Cu") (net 4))
 (segment (start 110.55 108.4955) (end 106.703 108.4955) (width 0.25) (layer "B.Cu") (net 4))
 (segment (start 181.0512 83.5354) (end 181.0512 82.2654) (width 0.25) (layer "B.Cu") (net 4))
 (segment (start 115.13 103.65) (end 107.9175 103.65) (width 0.25) (layer "B.Cu") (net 4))
 (segment (start 116.500989 105.020989) (end 115.13 103.65) (width 0.25) (layer "B.Cu") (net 4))
 (segment (start 106.703 108.4955) (end 104.8875 106.68) (width 0.25) (layer "B.Cu") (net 4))
 (segment (start 191.2112 83.5354) (end 187.062189 79.386389) (width 0.25) (layer "B.Cu") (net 4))
 (segment (start 107.9175 103.65) (end 104.8875 106.68) (width 0.25) (layer "B.Cu") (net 4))
 (segment (start 121.46 80.0725) (end 122.6675 81.28) (width 0.25) (layer "B.Cu") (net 31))
 (segment (start 121.46 77.44) (end 121.46 80.0725) (width 0.25) (layer "B.Cu") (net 31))
 (segment (start 166.9676 79.512) (end 167.3676 79.912) (width 0.25) (layer "B.Cu") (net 5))
 (segment (start 159.8676 79.512) (end 166.9676 79.512) (width 0.25) (layer "B.Cu") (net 5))
 (segment (start 146.8476 84.092) (end 146.8476 83.632) (width 0.25) (layer "B.Cu") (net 27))
 (segment (start 107.3775 75.4825) (end 108.44 74.42) (width 0.25) (layer "B.Cu") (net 27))
 (segment (start 146.8476 83.632) (end 147.8076 82.672) (width 0.25) (layer "B.Cu") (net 27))
 (segment (start 132.8275 75.4175) (end 132.8275 81.28) (width 0.25) (layer "B.Cu") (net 27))
 (segment (start 168.8176 82.672) (end 171.2351 85.0895) (width 0.25) (layer "B.Cu") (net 27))
 (segment (start 147.8076 82.672) (end 168.8176 82.672) (width 0.25) (layer "B.Cu") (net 27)))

